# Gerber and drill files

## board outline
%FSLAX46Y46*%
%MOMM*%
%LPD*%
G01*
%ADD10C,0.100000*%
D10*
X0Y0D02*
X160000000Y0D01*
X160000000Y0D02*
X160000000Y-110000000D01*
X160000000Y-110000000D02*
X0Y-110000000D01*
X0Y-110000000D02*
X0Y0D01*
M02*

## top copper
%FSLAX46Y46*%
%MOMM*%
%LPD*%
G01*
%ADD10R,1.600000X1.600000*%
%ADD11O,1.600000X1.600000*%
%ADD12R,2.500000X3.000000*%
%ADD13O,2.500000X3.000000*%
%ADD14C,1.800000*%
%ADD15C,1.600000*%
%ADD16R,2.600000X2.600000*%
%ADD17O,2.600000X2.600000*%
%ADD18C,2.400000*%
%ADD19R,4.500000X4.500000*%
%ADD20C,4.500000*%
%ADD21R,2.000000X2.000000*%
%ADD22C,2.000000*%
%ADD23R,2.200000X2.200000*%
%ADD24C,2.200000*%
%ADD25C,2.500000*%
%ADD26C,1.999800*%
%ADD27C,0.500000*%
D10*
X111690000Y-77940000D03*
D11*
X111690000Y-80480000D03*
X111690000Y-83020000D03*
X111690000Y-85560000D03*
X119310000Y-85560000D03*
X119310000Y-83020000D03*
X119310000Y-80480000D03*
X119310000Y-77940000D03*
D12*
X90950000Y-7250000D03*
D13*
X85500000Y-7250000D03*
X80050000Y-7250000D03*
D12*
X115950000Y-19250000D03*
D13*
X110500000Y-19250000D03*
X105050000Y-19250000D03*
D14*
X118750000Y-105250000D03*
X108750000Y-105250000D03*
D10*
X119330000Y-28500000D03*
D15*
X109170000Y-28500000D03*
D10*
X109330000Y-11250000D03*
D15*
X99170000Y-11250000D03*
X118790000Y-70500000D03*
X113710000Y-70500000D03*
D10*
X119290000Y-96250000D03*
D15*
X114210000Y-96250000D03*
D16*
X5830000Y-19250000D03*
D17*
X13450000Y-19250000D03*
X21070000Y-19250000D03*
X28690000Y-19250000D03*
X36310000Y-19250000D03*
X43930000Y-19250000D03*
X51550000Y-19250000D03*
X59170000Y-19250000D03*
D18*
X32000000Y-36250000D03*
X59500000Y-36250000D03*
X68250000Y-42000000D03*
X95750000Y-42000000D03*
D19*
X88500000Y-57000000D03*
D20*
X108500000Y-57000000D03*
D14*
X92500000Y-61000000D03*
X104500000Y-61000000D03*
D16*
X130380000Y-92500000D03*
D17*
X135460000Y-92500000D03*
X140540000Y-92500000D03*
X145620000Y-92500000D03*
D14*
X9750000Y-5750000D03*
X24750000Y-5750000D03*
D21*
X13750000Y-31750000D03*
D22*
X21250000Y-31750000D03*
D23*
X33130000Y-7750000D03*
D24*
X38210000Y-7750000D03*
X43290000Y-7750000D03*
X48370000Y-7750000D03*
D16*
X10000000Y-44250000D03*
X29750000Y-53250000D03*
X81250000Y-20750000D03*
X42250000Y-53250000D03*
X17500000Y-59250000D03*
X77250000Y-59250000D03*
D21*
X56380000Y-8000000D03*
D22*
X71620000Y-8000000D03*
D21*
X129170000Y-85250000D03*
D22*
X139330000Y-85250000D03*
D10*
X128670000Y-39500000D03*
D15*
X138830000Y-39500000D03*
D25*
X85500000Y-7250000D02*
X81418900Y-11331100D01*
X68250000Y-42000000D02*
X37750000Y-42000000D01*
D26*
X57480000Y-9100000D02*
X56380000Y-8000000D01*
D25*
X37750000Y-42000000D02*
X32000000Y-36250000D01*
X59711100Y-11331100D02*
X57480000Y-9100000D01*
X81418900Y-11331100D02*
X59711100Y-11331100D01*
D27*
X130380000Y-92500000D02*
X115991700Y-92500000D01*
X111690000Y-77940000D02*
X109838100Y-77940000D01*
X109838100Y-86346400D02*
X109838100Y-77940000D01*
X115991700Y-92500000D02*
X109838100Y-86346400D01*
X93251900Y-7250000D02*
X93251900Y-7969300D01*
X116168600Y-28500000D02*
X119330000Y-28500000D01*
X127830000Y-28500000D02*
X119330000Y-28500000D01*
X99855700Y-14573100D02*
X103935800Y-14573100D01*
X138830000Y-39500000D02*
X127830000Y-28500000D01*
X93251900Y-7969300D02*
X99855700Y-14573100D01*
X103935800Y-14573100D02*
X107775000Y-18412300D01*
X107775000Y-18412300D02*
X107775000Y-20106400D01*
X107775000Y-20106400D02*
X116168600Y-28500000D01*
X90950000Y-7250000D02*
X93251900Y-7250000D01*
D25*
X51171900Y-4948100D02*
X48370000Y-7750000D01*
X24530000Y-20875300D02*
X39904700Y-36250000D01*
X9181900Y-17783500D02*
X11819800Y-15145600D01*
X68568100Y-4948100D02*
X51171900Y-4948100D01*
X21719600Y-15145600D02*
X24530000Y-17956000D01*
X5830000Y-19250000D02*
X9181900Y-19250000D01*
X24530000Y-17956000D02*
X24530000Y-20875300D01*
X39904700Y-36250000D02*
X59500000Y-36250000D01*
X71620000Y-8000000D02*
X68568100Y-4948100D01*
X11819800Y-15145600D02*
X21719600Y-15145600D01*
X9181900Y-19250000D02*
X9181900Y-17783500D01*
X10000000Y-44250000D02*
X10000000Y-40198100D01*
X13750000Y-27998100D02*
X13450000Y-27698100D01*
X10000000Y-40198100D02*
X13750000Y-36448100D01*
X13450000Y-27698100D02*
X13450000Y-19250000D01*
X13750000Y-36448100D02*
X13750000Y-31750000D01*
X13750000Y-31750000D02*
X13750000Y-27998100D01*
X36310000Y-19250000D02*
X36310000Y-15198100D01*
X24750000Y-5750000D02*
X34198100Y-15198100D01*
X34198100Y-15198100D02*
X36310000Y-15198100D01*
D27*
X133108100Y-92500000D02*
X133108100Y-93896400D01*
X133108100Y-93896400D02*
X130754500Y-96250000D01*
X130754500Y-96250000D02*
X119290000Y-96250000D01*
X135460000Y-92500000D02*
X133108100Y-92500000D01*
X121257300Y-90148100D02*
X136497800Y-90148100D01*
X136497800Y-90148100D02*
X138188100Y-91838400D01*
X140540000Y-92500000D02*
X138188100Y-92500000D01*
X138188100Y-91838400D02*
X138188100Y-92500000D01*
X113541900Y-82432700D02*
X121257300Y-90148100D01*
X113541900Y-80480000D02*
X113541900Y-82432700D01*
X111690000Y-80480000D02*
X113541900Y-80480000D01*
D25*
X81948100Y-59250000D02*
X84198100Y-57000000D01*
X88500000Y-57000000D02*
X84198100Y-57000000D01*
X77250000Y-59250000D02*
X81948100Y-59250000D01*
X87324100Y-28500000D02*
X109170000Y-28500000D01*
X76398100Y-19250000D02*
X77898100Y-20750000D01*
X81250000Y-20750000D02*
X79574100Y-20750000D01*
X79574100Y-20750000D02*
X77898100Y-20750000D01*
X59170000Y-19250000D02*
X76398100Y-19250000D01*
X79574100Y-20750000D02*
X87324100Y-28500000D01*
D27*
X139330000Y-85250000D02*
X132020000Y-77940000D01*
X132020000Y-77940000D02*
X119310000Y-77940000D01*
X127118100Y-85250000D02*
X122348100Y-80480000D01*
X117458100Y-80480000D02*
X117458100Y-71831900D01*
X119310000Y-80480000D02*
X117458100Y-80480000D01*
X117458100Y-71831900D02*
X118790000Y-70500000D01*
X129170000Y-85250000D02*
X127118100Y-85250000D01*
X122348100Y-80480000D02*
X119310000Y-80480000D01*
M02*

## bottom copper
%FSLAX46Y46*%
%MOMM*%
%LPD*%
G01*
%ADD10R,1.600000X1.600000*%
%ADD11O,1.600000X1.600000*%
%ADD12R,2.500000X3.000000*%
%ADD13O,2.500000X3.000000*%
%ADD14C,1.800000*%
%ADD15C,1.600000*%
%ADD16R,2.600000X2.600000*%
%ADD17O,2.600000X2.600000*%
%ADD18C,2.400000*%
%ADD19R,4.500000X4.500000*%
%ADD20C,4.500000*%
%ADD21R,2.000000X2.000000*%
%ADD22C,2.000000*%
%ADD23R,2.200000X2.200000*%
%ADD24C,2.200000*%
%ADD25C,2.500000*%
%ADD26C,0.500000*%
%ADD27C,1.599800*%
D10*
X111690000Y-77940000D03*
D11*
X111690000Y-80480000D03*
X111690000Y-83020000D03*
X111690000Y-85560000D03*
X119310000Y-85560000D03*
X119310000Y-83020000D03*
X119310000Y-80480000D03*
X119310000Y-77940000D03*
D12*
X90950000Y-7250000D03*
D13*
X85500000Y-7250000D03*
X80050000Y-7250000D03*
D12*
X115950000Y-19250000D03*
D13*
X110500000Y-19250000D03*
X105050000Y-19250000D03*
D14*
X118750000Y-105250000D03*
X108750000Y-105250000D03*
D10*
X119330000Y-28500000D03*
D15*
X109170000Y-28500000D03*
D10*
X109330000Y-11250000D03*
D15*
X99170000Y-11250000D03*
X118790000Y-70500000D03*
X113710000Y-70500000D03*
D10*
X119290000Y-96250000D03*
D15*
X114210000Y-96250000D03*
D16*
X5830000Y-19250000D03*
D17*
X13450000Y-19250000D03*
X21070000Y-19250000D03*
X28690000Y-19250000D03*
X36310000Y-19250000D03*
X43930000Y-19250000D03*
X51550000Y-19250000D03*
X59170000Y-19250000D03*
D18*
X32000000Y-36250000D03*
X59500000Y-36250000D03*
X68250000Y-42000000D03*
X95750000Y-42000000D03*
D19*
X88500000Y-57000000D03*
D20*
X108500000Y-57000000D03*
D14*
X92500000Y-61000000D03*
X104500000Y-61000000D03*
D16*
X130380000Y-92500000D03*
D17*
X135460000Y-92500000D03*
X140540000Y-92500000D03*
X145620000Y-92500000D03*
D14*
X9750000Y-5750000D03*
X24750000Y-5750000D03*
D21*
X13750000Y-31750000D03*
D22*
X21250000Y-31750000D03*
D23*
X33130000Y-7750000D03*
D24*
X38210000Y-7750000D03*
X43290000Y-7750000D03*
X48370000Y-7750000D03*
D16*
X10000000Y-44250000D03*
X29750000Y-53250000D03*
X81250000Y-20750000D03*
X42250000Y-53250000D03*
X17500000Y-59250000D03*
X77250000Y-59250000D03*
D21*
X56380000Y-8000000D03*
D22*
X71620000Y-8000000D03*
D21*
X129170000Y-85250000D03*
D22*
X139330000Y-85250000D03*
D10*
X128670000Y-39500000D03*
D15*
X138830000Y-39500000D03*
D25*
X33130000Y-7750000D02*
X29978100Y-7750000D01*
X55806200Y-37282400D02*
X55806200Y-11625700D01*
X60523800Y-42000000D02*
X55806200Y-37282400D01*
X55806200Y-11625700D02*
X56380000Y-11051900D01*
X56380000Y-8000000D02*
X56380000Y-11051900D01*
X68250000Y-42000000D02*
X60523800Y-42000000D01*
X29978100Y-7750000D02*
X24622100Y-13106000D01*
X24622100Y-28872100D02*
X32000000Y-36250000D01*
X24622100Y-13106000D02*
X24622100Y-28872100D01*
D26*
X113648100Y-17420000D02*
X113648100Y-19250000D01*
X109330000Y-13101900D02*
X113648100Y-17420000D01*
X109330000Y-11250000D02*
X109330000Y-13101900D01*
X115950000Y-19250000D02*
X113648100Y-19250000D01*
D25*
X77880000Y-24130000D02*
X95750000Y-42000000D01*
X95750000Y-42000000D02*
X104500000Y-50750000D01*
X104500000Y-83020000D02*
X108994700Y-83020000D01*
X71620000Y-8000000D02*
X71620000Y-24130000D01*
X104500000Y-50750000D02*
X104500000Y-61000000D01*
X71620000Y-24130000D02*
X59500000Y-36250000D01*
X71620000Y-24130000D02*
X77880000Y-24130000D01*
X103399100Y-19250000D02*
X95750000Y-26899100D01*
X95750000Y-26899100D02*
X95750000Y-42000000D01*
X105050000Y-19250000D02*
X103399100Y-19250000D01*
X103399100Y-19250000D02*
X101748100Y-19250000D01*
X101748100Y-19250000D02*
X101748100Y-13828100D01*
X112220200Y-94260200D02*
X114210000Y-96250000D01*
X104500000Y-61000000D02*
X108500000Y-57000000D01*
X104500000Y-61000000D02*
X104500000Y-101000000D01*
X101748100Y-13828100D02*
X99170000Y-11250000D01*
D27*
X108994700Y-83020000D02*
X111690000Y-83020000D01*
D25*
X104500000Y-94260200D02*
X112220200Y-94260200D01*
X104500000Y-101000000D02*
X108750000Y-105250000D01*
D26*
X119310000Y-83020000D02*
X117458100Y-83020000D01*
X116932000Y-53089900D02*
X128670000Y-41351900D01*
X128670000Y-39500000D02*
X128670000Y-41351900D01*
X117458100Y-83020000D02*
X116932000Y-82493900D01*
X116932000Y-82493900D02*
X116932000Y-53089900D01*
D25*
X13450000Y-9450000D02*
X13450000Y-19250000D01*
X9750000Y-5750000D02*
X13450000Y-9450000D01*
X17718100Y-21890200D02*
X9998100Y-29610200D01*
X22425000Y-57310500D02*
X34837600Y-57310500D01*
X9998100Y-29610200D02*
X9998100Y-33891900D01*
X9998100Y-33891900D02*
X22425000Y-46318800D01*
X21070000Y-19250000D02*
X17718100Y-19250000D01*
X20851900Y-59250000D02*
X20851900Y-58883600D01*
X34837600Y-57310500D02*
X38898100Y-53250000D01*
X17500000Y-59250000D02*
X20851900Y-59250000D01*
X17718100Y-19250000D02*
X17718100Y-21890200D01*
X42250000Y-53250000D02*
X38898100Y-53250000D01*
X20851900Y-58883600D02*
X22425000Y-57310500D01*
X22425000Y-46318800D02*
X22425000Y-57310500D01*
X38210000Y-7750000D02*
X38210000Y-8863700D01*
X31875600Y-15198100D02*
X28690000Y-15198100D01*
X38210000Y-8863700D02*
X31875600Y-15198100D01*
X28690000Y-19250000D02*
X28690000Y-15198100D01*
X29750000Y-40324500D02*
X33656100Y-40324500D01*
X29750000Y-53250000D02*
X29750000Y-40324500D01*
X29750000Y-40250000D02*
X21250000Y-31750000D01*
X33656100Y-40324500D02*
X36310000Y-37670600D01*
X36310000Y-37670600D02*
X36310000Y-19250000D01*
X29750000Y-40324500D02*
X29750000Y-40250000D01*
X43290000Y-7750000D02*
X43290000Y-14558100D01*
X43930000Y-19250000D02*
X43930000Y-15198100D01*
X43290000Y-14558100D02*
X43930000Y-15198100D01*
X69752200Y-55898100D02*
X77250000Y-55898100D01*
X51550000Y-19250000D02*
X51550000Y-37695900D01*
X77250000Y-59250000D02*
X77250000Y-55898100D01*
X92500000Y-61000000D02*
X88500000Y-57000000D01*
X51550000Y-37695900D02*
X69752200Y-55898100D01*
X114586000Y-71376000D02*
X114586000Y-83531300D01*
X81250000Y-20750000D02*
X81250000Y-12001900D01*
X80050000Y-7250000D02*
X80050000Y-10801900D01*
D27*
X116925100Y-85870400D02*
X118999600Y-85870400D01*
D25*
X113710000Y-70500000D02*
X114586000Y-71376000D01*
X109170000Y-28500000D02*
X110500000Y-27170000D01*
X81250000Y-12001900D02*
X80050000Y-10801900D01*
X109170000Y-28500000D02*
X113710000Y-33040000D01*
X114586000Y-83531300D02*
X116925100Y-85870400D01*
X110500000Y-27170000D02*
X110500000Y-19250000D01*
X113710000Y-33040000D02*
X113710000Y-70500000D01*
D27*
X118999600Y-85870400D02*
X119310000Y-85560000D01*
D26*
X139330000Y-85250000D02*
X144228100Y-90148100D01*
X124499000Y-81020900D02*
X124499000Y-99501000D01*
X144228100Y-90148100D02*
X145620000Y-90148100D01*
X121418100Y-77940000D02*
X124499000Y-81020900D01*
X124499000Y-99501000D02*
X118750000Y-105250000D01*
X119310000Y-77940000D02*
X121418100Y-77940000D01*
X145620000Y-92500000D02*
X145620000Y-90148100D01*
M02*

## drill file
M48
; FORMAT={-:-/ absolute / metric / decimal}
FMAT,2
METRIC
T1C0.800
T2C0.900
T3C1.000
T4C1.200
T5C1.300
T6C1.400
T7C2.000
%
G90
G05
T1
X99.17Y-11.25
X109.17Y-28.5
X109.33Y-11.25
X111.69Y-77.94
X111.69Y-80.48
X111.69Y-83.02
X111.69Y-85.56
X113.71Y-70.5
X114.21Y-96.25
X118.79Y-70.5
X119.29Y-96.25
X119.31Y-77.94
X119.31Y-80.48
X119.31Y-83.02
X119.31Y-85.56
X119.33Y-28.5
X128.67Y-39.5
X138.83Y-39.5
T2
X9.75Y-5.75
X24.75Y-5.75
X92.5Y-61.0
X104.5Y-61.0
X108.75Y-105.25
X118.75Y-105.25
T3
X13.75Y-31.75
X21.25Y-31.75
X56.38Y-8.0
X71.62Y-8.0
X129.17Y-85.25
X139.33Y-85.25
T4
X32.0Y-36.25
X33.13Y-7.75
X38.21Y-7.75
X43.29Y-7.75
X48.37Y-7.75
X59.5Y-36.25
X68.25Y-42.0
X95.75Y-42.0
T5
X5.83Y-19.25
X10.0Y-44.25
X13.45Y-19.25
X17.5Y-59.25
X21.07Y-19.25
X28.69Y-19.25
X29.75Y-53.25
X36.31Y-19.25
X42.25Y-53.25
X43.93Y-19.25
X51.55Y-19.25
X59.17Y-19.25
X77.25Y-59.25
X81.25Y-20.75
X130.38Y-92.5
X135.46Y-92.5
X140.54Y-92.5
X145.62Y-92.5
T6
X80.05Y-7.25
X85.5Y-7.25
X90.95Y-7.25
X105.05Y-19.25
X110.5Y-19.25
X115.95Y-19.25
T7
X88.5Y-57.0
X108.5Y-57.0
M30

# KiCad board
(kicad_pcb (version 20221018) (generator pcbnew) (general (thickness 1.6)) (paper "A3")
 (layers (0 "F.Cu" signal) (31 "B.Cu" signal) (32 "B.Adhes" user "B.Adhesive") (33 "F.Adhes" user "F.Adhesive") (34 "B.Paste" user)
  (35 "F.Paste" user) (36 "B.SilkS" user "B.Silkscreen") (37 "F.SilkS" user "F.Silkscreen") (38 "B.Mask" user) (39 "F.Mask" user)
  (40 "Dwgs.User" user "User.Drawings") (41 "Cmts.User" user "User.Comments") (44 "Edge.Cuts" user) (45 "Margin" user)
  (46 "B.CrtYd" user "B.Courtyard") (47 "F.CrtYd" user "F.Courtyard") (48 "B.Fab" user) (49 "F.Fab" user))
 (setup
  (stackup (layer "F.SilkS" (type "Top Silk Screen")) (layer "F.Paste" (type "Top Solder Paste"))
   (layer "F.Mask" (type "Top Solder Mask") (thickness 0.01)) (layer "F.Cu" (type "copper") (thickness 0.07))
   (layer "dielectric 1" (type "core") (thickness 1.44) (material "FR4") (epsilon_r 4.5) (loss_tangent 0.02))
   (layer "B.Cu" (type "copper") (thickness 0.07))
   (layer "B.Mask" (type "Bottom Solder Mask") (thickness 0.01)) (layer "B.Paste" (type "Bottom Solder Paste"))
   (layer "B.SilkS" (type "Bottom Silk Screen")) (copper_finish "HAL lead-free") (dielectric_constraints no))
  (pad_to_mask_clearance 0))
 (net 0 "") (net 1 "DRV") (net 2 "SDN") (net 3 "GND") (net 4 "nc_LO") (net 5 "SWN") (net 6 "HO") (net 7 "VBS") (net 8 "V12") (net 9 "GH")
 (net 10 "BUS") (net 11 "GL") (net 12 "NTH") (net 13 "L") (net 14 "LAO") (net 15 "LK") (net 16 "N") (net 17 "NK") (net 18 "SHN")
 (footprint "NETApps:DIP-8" (layer "F.Cu") (at 115.5 81.75)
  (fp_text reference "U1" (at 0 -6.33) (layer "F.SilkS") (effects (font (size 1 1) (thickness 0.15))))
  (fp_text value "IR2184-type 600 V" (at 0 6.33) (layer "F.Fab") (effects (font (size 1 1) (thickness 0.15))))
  (pad "1" thru_hole rect (at -3.81 -3.81) (size 1.6 1.6) (drill 0.8) (layers "*.Cu" "*.Mask") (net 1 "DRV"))
  (pad "2" thru_hole oval (at -3.81 -1.27) (size 1.6 1.6) (drill 0.8) (layers "*.Cu" "*.Mask") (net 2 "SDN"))
  (pad "3" thru_hole oval (at -3.81 1.27) (size 1.6 1.6) (drill 0.8) (layers "*.Cu" "*.Mask") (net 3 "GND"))
  (pad "4" thru_hole oval (at -3.81 3.81) (size 1.6 1.6) (drill 0.8) (layers "*.Cu" "*.Mask") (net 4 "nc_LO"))
  (pad "5" thru_hole oval (at 3.81 3.81) (size 1.6 1.6) (drill 0.8) (layers "*.Cu" "*.Mask") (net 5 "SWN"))
  (pad "6" thru_hole oval (at 3.81 1.27) (size 1.6 1.6) (drill 0.8) (layers "*.Cu" "*.Mask") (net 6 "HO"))
  (pad "7" thru_hole oval (at 3.81 -1.27) (size 1.6 1.6) (drill 0.8) (layers "*.Cu" "*.Mask") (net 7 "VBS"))
  (pad "8" thru_hole oval (at 3.81 -3.81) (size 1.6 1.6) (drill 0.8) (layers "*.Cu" "*.Mask") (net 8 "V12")))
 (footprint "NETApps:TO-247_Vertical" (layer "F.Cu") (at 85.5 7.25 180)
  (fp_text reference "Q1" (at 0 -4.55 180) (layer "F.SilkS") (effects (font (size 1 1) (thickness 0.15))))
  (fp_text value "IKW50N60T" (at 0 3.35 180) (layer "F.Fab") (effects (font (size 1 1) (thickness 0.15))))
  (pad "1" thru_hole rect (at -5.45 0) (size 2.5 3) (drill 1.4) (layers "*.Cu" "*.Mask") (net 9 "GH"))
  (pad "2" thru_hole oval (at 0 0) (size 2.5 3) (drill 1.4) (layers "*.Cu" "*.Mask") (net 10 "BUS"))
  (pad "3" thru_hole oval (at 5.45 0) (size 2.5 3) (drill 1.4) (layers "*.Cu" "*.Mask") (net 5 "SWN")))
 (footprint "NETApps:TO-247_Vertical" (layer "F.Cu") (at 110.5 19.25 180)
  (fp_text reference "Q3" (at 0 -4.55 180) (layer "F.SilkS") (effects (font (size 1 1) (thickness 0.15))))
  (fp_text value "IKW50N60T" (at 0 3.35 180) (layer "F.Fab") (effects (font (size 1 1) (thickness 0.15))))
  (pad "1" thru_hole rect (at -5.45 0) (size 2.5 3) (drill 1.4) (layers "*.Cu" "*.Mask") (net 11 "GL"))
  (pad "2" thru_hole oval (at 0 0) (size 2.5 3) (drill 1.4) (layers "*.Cu" "*.Mask") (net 5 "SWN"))
  (pad "3" thru_hole oval (at 5.45 0) (size 2.5 3) (drill 1.4) (layers "*.Cu" "*.Mask") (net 3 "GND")))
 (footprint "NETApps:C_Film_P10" (layer "F.Cu") (at 113.75 105.25 180)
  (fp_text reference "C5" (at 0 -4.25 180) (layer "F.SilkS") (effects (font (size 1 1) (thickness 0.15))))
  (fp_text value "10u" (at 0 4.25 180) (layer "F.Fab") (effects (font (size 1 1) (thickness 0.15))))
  (pad "1" thru_hole circle (at -5 0) (size 1.8 1.8) (drill 0.9) (layers "*.Cu" "*.Mask") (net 8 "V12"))
  (pad "2" thru_hole circle (at 5 0) (size 1.8 1.8) (drill 0.9) (layers "*.Cu" "*.Mask") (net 3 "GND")))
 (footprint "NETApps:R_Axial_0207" (layer "F.Cu") (at 114.25 28.5 180)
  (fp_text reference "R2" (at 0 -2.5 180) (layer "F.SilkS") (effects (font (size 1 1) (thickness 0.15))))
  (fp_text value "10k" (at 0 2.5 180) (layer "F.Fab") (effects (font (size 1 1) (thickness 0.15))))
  (pad "1" thru_hole rect (at -5.08 0) (size 1.6 1.6) (drill 0.8) (layers "*.Cu" "*.Mask") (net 9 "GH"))
  (pad "2" thru_hole circle (at 5.08 0) (size 1.6 1.6) (drill 0.8) (layers "*.Cu" "*.Mask") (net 5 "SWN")))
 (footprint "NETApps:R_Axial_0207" (layer "F.Cu") (at 104.25 11.25 180)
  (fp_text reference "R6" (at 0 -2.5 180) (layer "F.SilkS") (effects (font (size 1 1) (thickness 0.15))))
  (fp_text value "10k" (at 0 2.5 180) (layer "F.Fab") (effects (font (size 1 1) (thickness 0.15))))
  (pad "1" thru_hole rect (at -5.08 0) (size 1.6 1.6) (drill 0.8) (layers "*.Cu" "*.Mask") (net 11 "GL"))
  (pad "2" thru_hole circle (at 5.08 0) (size 1.6 1.6) (drill 0.8) (layers "*.Cu" "*.Mask") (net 3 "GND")))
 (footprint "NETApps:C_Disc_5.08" (layer "F.Cu") (at 116.25 70.5 180)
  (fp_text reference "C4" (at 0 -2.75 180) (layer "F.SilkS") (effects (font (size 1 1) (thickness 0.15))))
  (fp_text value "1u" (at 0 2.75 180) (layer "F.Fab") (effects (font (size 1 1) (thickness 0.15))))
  (pad "1" thru_hole circle (at -2.54 0) (size 1.6 1.6) (drill 0.8) (layers "*.Cu" "*.Mask") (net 7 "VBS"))
  (pad "2" thru_hole circle (at 2.54 0) (size 1.6 1.6) (drill 0.8) (layers "*.Cu" "*.Mask") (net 5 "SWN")))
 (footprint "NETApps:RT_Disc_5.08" (layer "F.Cu") (at 116.75 96.25 180)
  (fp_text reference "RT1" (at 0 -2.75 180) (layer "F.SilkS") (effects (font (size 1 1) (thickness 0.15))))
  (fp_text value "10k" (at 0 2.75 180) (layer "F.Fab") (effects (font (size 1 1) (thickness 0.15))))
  (pad "1" thru_hole rect (at -2.54 0) (size 1.6 1.6) (drill 0.8) (layers "*.Cu" "*.Mask") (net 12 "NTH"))
  (pad "2" thru_hole circle (at 2.54 0) (size 1.6 1.6) (drill 0.8) (layers "*.Cu" "*.Mask") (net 3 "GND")))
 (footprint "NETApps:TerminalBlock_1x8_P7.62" (layer "F.Cu") (at 32.5 19.25)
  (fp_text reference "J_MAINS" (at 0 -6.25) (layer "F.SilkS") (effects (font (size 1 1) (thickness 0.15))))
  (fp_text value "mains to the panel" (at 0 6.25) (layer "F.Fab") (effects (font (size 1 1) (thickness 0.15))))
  (pad "1" thru_hole rect (at -26.67 0) (size 2.6 2.6) (drill 1.3) (layers "*.Cu" "*.Mask") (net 3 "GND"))
  (pad "2" thru_hole oval (at -19.05 0) (size 2.6 2.6) (drill 1.3) (layers "*.Cu" "*.Mask") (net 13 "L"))
  (pad "3" thru_hole oval (at -11.43 0) (size 2.6 2.6) (drill 1.3) (layers "*.Cu" "*.Mask") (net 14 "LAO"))
  (pad "4" thru_hole oval (at -3.81 0) (size 2.6 2.6) (drill 1.3) (layers "*.Cu" "*.Mask") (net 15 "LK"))
  (pad "5" thru_hole oval (at 3.81 0) (size 2.6 2.6) (drill 1.3) (layers "*.Cu" "*.Mask") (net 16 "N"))
  (pad "6" thru_hole oval (at 11.43 0) (size 2.6 2.6) (drill 1.3) (layers "*.Cu" "*.Mask") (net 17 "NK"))
  (pad "7" thru_hole oval (at 19.05 0) (size 2.6 2.6) (drill 1.3) (layers "*.Cu" "*.Mask") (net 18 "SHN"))
  (pad "8" thru_hole oval (at 26.67 0) (size 2.6 2.6) (drill 1.3) (layers "*.Cu" "*.Mask") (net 5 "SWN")))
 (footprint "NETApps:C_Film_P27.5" (layer "F.Cu") (at 45.75 36.25)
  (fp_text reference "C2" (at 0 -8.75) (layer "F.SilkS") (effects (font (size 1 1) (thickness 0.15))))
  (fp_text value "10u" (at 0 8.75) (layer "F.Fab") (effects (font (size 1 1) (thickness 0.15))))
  (pad "1" thru_hole circle (at -13.75 0) (size 2.4 2.4) (drill 1.2) (layers "*.Cu" "*.Mask") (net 10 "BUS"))
  (pad "2" thru_hole circle (at 13.75 0) (size 2.4 2.4) (drill 1.2) (layers "*.Cu" "*.Mask") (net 3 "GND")))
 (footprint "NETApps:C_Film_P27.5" (layer "F.Cu") (at 82 42)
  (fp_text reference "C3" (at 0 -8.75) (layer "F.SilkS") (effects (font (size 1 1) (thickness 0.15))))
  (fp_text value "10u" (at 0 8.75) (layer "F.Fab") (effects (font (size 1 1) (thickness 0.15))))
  (pad "1" thru_hole circle (at -13.75 0) (size 2.4 2.4) (drill 1.2) (layers "*.Cu" "*.Mask") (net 10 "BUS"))
  (pad "2" thru_hole circle (at 13.75 0) (size 2.4 2.4) (drill 1.2) (layers "*.Cu" "*.Mask") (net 3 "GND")))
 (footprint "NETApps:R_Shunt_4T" (layer "F.Cu") (at 98.5 57)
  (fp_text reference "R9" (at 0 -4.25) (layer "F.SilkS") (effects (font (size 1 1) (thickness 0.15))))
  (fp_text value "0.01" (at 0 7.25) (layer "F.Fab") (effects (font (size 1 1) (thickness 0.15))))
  (pad "1" thru_hole rect (at -10 0) (size 4.5 4.5) (drill 2) (layers "*.Cu" "*.Mask") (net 18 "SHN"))
  (pad "2" thru_hole circle (at 10 0) (size 4.5 4.5) (drill 2) (layers "*.Cu" "*.Mask") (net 3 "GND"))
  (pad "3" thru_hole circle (at -6 4) (size 1.8 1.8) (drill 0.9) (layers "*.Cu" "*.Mask") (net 18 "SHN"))
  (pad "4" thru_hole circle (at 6 4) (size 1.8 1.8) (drill 0.9) (layers "*.Cu" "*.Mask") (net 3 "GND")))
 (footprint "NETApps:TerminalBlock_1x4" (layer "F.Cu") (at 138 92.5)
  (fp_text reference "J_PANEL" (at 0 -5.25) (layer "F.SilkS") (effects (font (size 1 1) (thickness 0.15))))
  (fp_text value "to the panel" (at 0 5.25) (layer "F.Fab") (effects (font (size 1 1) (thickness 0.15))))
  (pad "1" thru_hole rect (at -7.62 0) (size 2.6 2.6) (drill 1.3) (layers "*.Cu" "*.Mask") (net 1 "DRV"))
  (pad "2" thru_hole oval (at -2.54 0) (size 2.6 2.6) (drill 1.3) (layers "*.Cu" "*.Mask") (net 12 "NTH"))
  (pad "3" thru_hole oval (at 2.54 0) (size 2.6 2.6) (drill 1.3) (layers "*.Cu" "*.Mask") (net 2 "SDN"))
  (pad "4" thru_hole oval (at 7.62 0) (size 2.6 2.6) (drill 1.3) (layers "*.Cu" "*.Mask") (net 8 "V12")))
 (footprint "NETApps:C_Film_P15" (layer "F.Cu") (at 17.25 5.75)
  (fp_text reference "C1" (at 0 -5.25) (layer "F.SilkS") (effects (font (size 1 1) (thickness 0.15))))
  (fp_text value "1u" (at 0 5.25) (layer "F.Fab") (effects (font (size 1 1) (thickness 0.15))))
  (pad "1" thru_hole circle (at -7.5 0) (size 1.8 1.8) (drill 0.9) (layers "*.Cu" "*.Mask") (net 13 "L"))
  (pad "2" thru_hole circle (at 7.5 0) (size 1.8 1.8) (drill 0.9) (layers "*.Cu" "*.Mask") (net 16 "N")))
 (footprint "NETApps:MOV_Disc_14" (layer "F.Cu") (at 17.5 31.75)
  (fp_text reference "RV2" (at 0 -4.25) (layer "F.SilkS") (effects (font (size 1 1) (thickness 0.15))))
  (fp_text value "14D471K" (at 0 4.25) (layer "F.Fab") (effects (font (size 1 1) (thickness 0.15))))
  (pad "1" thru_hole rect (at -3.75 0) (size 2 2) (drill 1) (layers "*.Cu" "*.Mask") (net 13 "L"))
  (pad "2" thru_hole circle (at 3.75 0) (size 2 2) (drill 1) (layers "*.Cu" "*.Mask") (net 16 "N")))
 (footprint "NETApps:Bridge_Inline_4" (layer "F.Cu") (at 40.75 7.75)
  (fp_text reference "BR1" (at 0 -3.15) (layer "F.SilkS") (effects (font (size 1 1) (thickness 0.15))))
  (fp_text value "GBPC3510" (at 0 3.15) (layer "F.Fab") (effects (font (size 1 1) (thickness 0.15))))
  (pad "1" thru_hole rect (at -7.62 0) (size 2.2 2.2) (drill 1.2) (layers "*.Cu" "*.Mask") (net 10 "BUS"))
  (pad "2" thru_hole circle (at -2.54 0) (size 2.2 2.2) (drill 1.2) (layers "*.Cu" "*.Mask") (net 15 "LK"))
  (pad "3" thru_hole circle (at 2.54 0) (size 2.2 2.2) (drill 1.2) (layers "*.Cu" "*.Mask") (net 17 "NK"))
  (pad "4" thru_hole circle (at 7.62 0) (size 2.2 2.2) (drill 1.2) (layers "*.Cu" "*.Mask") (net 3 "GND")))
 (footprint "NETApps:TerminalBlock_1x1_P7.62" (layer "F.Cu") (at 10 44.25)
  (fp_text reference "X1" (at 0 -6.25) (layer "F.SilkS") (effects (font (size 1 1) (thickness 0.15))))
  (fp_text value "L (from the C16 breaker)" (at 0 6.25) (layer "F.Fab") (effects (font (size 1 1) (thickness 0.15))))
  (pad "1" thru_hole rect (at 0 0) (size 2.6 2.6) (drill 1.3) (layers "*.Cu" "*.Mask") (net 13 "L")))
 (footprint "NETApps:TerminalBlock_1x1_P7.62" (layer "F.Cu") (at 29.75 53.25)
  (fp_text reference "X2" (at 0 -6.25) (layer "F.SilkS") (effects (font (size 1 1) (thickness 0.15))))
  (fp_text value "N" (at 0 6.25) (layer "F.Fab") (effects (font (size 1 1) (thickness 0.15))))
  (pad "1" thru_hole rect (at 0 0) (size 2.6 2.6) (drill 1.3) (layers "*.Cu" "*.Mask") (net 16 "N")))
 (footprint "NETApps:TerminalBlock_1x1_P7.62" (layer "F.Cu") (at 81.25 20.75)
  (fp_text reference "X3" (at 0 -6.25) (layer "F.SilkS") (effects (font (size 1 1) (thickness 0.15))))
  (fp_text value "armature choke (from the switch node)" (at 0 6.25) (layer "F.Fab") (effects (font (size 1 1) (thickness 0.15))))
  (pad "1" thru_hole rect (at 0 0) (size 2.6 2.6) (drill 1.3) (layers "*.Cu" "*.Mask") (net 5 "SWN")))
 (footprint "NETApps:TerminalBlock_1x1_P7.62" (layer "F.Cu") (at 42.25 53.25)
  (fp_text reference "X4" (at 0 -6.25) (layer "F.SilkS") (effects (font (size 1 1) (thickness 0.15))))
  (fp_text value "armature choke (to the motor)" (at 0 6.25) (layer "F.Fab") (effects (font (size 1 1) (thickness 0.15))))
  (pad "1" thru_hole rect (at 0 0) (size 2.6 2.6) (drill 1.3) (layers "*.Cu" "*.Mask") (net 14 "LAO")))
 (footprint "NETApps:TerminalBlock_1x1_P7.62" (layer "F.Cu") (at 17.5 59.25)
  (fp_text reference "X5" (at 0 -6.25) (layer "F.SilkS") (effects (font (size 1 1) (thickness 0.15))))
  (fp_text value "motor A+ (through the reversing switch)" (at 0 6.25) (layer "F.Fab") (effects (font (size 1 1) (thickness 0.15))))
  (pad "1" thru_hole rect (at 0 0) (size 2.6 2.6) (drill 1.3) (layers "*.Cu" "*.Mask") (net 14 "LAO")))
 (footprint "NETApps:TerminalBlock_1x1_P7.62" (layer "F.Cu") (at 77.25 59.25)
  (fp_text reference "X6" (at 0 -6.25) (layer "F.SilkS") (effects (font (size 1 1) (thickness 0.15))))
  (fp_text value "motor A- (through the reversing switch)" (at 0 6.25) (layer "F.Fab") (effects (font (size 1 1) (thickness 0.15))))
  (pad "1" thru_hole rect (at 0 0) (size 2.6 2.6) (drill 1.3) (layers "*.Cu" "*.Mask") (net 18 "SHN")))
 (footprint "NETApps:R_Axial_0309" (layer "F.Cu") (at 64 8)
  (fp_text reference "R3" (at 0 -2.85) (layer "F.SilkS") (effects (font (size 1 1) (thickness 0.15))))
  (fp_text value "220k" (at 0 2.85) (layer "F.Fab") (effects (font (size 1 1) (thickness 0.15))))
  (pad "1" thru_hole rect (at -7.62 0) (size 2 2) (drill 1) (layers "*.Cu" "*.Mask") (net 10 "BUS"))
  (pad "2" thru_hole circle (at 7.62 0) (size 2 2) (drill 1) (layers "*.Cu" "*.Mask") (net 3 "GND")))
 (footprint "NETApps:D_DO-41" (layer "F.Cu") (at 134.25 85.25)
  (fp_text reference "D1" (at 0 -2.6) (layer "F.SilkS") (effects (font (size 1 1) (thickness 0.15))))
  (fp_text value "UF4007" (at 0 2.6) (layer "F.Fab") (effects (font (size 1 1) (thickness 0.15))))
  (pad "1" thru_hole rect (at -5.08 0) (size 2 2) (drill 1) (layers "*.Cu" "*.Mask") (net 7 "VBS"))
  (pad "2" thru_hole circle (at 5.08 0) (size 2 2) (drill 1) (layers "*.Cu" "*.Mask") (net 8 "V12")))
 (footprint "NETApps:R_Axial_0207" (layer "F.Cu") (at 133.75 39.5)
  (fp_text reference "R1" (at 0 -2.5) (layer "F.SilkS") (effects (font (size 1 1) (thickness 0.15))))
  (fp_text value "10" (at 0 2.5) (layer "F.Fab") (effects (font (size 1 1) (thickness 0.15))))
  (pad "1" thru_hole rect (at -5.08 0) (size 1.6 1.6) (drill 0.8) (layers "*.Cu" "*.Mask") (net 6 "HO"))
  (pad "2" thru_hole circle (at 5.08 0) (size 1.6 1.6) (drill 0.8) (layers "*.Cu" "*.Mask") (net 9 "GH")))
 (gr_line (start 0 0) (end 160 0) (stroke (width 0.1) (type solid)) (layer "Edge.Cuts"))
 (gr_line (start 160 0) (end 160 110) (stroke (width 0.1) (type solid)) (layer "Edge.Cuts"))
 (gr_line (start 160 110) (end 0 110) (stroke (width 0.1) (type solid)) (layer "Edge.Cuts"))
 (gr_line (start 0 110) (end 0 0) (stroke (width 0.1) (type solid)) (layer "Edge.Cuts"))
 (segment (start 85.5 7.25) (end 81.4189 11.3311) (width 2.5) (layer "F.Cu") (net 10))
 (segment locked (start 68.25 42) (end 37.75 42) (width 2.5) (layer "F.Cu") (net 10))
 (segment (start 57.48 9.1) (end 56.38 8) (width 1.9998) (layer "F.Cu") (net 10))
 (segment locked (start 37.75 42) (end 32 36.25) (width 2.5) (layer "F.Cu") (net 10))
 (segment (start 59.7111 11.3311) (end 57.48 9.1) (width 2.5) (layer "F.Cu") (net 10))
 (segment (start 81.4189 11.3311) (end 59.7111 11.3311) (width 2.5) (layer "F.Cu") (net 10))
 (segment locked (start 33.13 7.75) (end 29.9781 7.75) (width 2.5) (layer "B.Cu") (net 10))
 (segment locked (start 55.8062 37.2824) (end 55.8062 11.6257) (width 2.5) (layer "B.Cu") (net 10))
 (segment locked (start 60.5238 42) (end 55.8062 37.2824) (width 2.5) (layer "B.Cu") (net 10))
 (segment locked (start 55.8062 11.6257) (end 56.38 11.0519) (width 2.5) (layer "B.Cu") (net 10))
 (segment locked (start 56.38 8) (end 56.38 11.0519) (width 2.5) (layer "B.Cu") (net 10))
 (segment locked (start 68.25 42) (end 60.5238 42) (width 2.5) (layer "B.Cu") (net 10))
 (segment locked (start 29.9781 7.75) (end 24.6221 13.106) (width 2.5) (layer "B.Cu") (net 10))
 (segment locked (start 24.6221 28.8721) (end 32 36.25) (width 2.5) (layer "B.Cu") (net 10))
 (segment locked (start 24.6221 13.106) (end 24.6221 28.8721) (width 2.5) (layer "B.Cu") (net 10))
 (segment (start 130.38 92.5) (end 115.9917 92.5) (width 0.5) (layer "F.Cu") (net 1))
 (segment (start 111.69 77.94) (end 109.8381 77.94) (width 0.5) (layer "F.Cu") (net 1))
 (segment (start 109.8381 86.3464) (end 109.8381 77.94) (width 0.5) (layer "F.Cu") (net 1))
 (segment (start 115.9917 92.5) (end 109.8381 86.3464) (width 0.5) (layer "F.Cu") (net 1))
 (segment (start 93.2519 7.25) (end 93.2519 7.9693) (width 0.5) (layer "F.Cu") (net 9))
 (segment (start 116.1686 28.5) (end 119.33 28.5) (width 0.5) (layer "F.Cu") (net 9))
 (segment (start 127.83 28.5) (end 119.33 28.5) (width 0.5) (layer "F.Cu") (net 9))
 (segment (start 99.8557 14.5731) (end 103.9358 14.5731) (width 0.5) (layer "F.Cu") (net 9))
 (segment (start 138.83 39.5) (end 127.83 28.5) (width 0.5) (layer "F.Cu") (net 9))
 (segment (start 93.2519 7.9693) (end 99.8557 14.5731) (width 0.5) (layer "F.Cu") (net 9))
 (segment (start 103.9358 14.5731) (end 107.775 18.4123) (width 0.5) (layer "F.Cu") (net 9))
 (segment (start 107.775 18.4123) (end 107.775 20.1064) (width 0.5) (layer "F.Cu") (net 9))
 (segment (start 107.775 20.1064) (end 116.1686 28.5) (width 0.5) (layer "F.Cu") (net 9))
 (segment (start 90.95 7.25) (end 93.2519 7.25) (width 0.5) (layer "F.Cu") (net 9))
 (segment (start 113.6481 17.42) (end 113.6481 19.25) (width 0.5) (layer "B.Cu") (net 11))
 (segment (start 109.33 13.1019) (end 113.6481 17.42) (width 0.5) (layer "B.Cu") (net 11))
 (segment (start 109.33 11.25) (end 109.33 13.1019) (width 0.5) (layer "B.Cu") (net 11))
 (segment (start 115.95 19.25) (end 113.6481 19.25) (width 0.5) (layer "B.Cu") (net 11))
 (segment locked (start 51.1719 4.9481) (end 48.37 7.75) (width 2.5) (layer "F.Cu") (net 3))
 (segment locked (start 24.53 20.8753) (end 39.9047 36.25) (width 2.5) (layer "F.Cu") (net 3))
 (segment locked (start 9.1819 17.7835) (end 11.8198 15.1456) (width 2.5) (layer "F.Cu") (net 3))
 (segment locked (start 68.5681 4.9481) (end 51.1719 4.9481) (width 2.5) (layer "F.Cu") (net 3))
 (segment locked (start 21.7196 15.1456) (end 24.53 17.956) (width 2.5) (layer "F.Cu") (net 3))
 (segment locked (start 5.83 19.25) (end 9.1819 19.25) (width 2.5) (layer "F.Cu") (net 3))
 (segment locked (start 24.53 17.956) (end 24.53 20.8753) (width 2.5) (layer "F.Cu") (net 3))
 (segment locked (start 39.9047 36.25) (end 59.5 36.25) (width 2.5) (layer "F.Cu") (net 3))
 (segment locked (start 71.62 8) (end 68.5681 4.9481) (width 2.5) (layer "F.Cu") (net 3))
 (segment locked (start 11.8198 15.1456) (end 21.7196 15.1456) (width 2.5) (layer "F.Cu") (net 3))
 (segment locked (start 9.1819 19.25) (end 9.1819 17.7835) (width 2.5) (layer "F.Cu") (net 3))
 (segment locked (start 77.88 24.13) (end 95.75 42) (width 2.5) (layer "B.Cu") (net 3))
 (segment locked (start 95.75 42) (end 104.5 50.75) (width 2.5) (layer "B.Cu") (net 3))
 (segment (start 104.5 83.02) (end 108.9947 83.02) (width 2.5) (layer "B.Cu") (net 3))
 (segment locked (start 71.62 8) (end 71.62 24.13) (width 2.5) (layer "B.Cu") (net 3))
 (segment locked (start 104.5 50.75) (end 104.5 61) (width 2.5) (layer "B.Cu") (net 3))
 (segment locked (start 71.62 24.13) (end 59.5 36.25) (width 2.5) (layer "B.Cu") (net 3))
 (segment locked (start 71.62 24.13) (end 77.88 24.13) (width 2.5) (layer "B.Cu") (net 3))
 (segment locked (start 103.3991 19.25) (end 95.75 26.8991) (width 2.5) (layer "B.Cu") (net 3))
 (segment locked (start 95.75 26.8991) (end 95.75 42) (width 2.5) (layer "B.Cu") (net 3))
 (segment locked (start 105.05 19.25) (end 103.3991 19.25) (width 2.5) (layer "B.Cu") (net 3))
 (segment locked (start 103.3991 19.25) (end 101.7481 19.25) (width 2.5) (layer "B.Cu") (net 3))
 (segment locked (start 101.7481 19.25) (end 101.7481 13.8281) (width 2.5) (layer "B.Cu") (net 3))
 (segment (start 112.2202 94.2602) (end 114.21 96.25) (width 2.5) (layer "B.Cu") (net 3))
 (segment locked (start 104.5 61) (end 108.5 57) (width 2.5) (layer "B.Cu") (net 3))
 (segment locked (start 104.5 61) (end 104.5 101) (width 2.5) (layer "B.Cu") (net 3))
 (segment locked (start 101.7481 13.8281) (end 99.17 11.25) (width 2.5) (layer "B.Cu") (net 3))
 (segment (start 108.9947 83.02) (end 111.69 83.02) (width 1.5998) (layer "B.Cu") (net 3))
 (segment (start 104.5 94.2602) (end 112.2202 94.2602) (width 2.5) (layer "B.Cu") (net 3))
 (segment locked (start 104.5 101) (end 108.75 105.25) (width 2.5) (layer "B.Cu") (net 3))
 (segment (start 119.31 83.02) (end 117.4581 83.02) (width 0.5) (layer "B.Cu") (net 6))
 (segment (start 116.932 53.0899) (end 128.67 41.3519) (width 0.5) (layer "B.Cu") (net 6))
 (segment (start 128.67 39.5) (end 128.67 41.3519) (width 0.5) (layer "B.Cu") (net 6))
 (segment (start 117.4581 83.02) (end 116.932 82.4939) (width 0.5) (layer "B.Cu") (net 6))
 (segment (start 116.932 82.4939) (end 116.932 53.0899) (width 0.5) (layer "B.Cu") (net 6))
 (segment locked (start 10 44.25) (end 10 40.1981) (width 2.5) (layer "F.Cu") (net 13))
 (segment locked (start 13.75 27.9981) (end 13.45 27.6981) (width 2.5) (layer "F.Cu") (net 13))
 (segment locked (start 10 40.1981) (end 13.75 36.4481) (width 2.5) (layer "F.Cu") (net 13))
 (segment locked (start 13.45 27.6981) (end 13.45 19.25) (width 2.5) (layer "F.Cu") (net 13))
 (segment locked (start 13.75 36.4481) (end 13.75 31.75) (width 2.5) (layer "F.Cu") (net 13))
 (segment locked (start 13.75 31.75) (end 13.75 27.9981) (width 2.5) (layer "F.Cu") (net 13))
 (segment locked (start 13.45 9.45) (end 13.45 19.25) (width 2.5) (layer "B.Cu") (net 13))
 (segment locked (start 9.75 5.75) (end 13.45 9.45) (width 2.5) (layer "B.Cu") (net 13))
 (segment locked (start 17.7181 21.8902) (end 9.9981 29.6102) (width 2.5) (layer "B.Cu") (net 14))
 (segment locked (start 22.425 57.3105) (end 34.8376 57.3105) (width 2.5) (layer "B.Cu") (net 14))
 (segment locked (start 9.9981 29.6102) (end 9.9981 33.8919) (width 2.5) (layer "B.Cu") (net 14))
 (segment locked (start 9.9981 33.8919) (end 22.425 46.3188) (width 2.5) (layer "B.Cu") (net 14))
 (segment locked (start 21.07 19.25) (end 17.7181 19.25) (width 2.5) (layer "B.Cu") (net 14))
 (segment locked (start 20.8519 59.25) (end 20.8519 58.8836) (width 2.5) (layer "B.Cu") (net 14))
 (segment locked (start 34.8376 57.3105) (end 38.8981 53.25) (width 2.5) (layer "B.Cu") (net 14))
 (segment locked (start 17.5 59.25) (end 20.8519 59.25) (width 2.5) (layer "B.Cu") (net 14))
 (segment locked (start 17.7181 19.25) (end 17.7181 21.8902) (width 2.5) (layer "B.Cu") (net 14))
 (segment locked (start 42.25 53.25) (end 38.8981 53.25) (width 2.5) (layer "B.Cu") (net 14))
 (segment locked (start 20.8519 58.8836) (end 22.425 57.3105) (width 2.5) (layer "B.Cu") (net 14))
 (segment locked (start 22.425 46.3188) (end 22.425 57.3105) (width 2.5) (layer "B.Cu") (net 14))
 (segment locked (start 38.21 7.75) (end 38.21 8.8637) (width 2.5) (layer "B.Cu") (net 15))
 (segment locked (start 31.8756 15.1981) (end 28.69 15.1981) (width 2.5) (layer "B.Cu") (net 15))
 (segment locked (start 38.21 8.8637) (end 31.8756 15.1981) (width 2.5) (layer "B.Cu") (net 15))
 (segment locked (start 28.69 19.25) (end 28.69 15.1981) (width 2.5) (layer "B.Cu") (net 15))
 (segment locked (start 36.31 19.25) (end 36.31 15.1981) (width 2.5) (layer "F.Cu") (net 16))
 (segment locked (start 24.75 5.75) (end 34.1981 15.1981) (width 2.5) (layer "F.Cu") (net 16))
 (segment locked (start 34.1981 15.1981) (end 36.31 15.1981) (width 2.5) (layer "F.Cu") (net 16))
 (segment locked (start 29.75 40.3245) (end 33.6561 40.3245) (width 2.5) (layer "B.Cu") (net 16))
 (segment locked (start 29.75 53.25) (end 29.75 40.3245) (width 2.5) (layer "B.Cu") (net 16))
 (segment locked (start 29.75 40.25) (end 21.25 31.75) (width 2.5) (layer "B.Cu") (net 16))
 (segment locked (start 33.6561 40.3245) (end 36.31 37.6706) (width 2.5) (layer "B.Cu") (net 16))
 (segment locked (start 36.31 37.6706) (end 36.31 19.25) (width 2.5) (layer "B.Cu") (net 16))
 (segment locked (start 29.75 40.3245) (end 29.75 40.25) (width 2.5) (layer "B.Cu") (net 16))
 (segment locked (start 43.29 7.75) (end 43.29 14.5581) (width 2.5) (layer "B.Cu") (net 17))
 (segment locked (start 43.93 19.25) (end 43.93 15.1981) (width 2.5) (layer "B.Cu") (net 17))
 (segment locked (start 43.29 14.5581) (end 43.93 15.1981) (width 2.5) (layer "B.Cu") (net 17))
 (segment (start 133.1081 92.5) (end 133.1081 93.8964) (width 0.5) (layer "F.Cu") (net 12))
 (segment (start 133.1081 93.8964) (end 130.7545 96.25) (width 0.5) (layer "F.Cu") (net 12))
 (segment (start 130.7545 96.25) (end 119.29 96.25) (width 0.5) (layer "F.Cu") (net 12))
 (segment (start 135.46 92.5) (end 133.1081 92.5) (width 0.5) (layer "F.Cu") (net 12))
 (segment (start 121.2573 90.1481) (end 136.4978 90.1481) (width 0.5) (layer "F.Cu") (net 2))
 (segment (start 136.4978 90.1481) (end 138.1881 91.8384) (width 0.5) (layer "F.Cu") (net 2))
 (segment (start 140.54 92.5) (end 138.1881 92.5) (width 0.5) (layer "F.Cu") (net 2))
 (segment (start 138.1881 91.8384) (end 138.1881 92.5) (width 0.5) (layer "F.Cu") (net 2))
 (segment (start 113.5419 82.4327) (end 121.2573 90.1481) (width 0.5) (layer "F.Cu") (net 2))
 (segment (start 113.5419 80.48) (end 113.5419 82.4327) (width 0.5) (layer "F.Cu") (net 2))
 (segment (start 111.69 80.48) (end 113.5419 80.48) (width 0.5) (layer "F.Cu") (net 2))
 (segment locked (start 81.9481 59.25) (end 84.1981 57) (width 2.5) (layer "F.Cu") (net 18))
 (segment locked (start 88.5 57) (end 84.1981 57) (width 2.5) (layer "F.Cu") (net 18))
 (segment locked (start 77.25 59.25) (end 81.9481 59.25) (width 2.5) (layer "F.Cu") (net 18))
 (segment locked (start 69.7522 55.8981) (end 77.25 55.8981) (width 2.5) (layer "B.Cu") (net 18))
 (segment locked (start 51.55 19.25) (end 51.55 37.6959) (width 2.5) (layer "B.Cu") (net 18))
 (segment locked (start 77.25 59.25) (end 77.25 55.8981) (width 2.5) (layer "B.Cu") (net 18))
 (segment locked (start 92.5 61) (end 88.5 57) (width 2.5) (layer "B.Cu") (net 18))
 (segment locked (start 51.55 37.6959) (end 69.7522 55.8981) (width 2.5) (layer "B.Cu") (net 18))
 (segment locked (start 87.3241 28.5) (end 109.17 28.5) (width 2.5) (layer "F.Cu") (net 5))
 (segment locked (start 76.3981 19.25) (end 77.8981 20.75) (width 2.5) (layer "F.Cu") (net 5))
 (segment locked (start 81.25 20.75) (end 79.5741 20.75) (width 2.5) (layer "F.Cu") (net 5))
 (segment locked (start 79.5741 20.75) (end 77.8981 20.75) (width 2.5) (layer "F.Cu") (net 5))
 (segment locked (start 59.17 19.25) (end 76.3981 19.25) (width 2.5) (layer "F.Cu") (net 5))
 (segment locked (start 79.5741 20.75) (end 87.3241 28.5) (width 2.5) (layer "F.Cu") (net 5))
 (segment (start 114.586 71.376) (end 114.586 83.5313) (width 2.5) (layer "B.Cu") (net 5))
 (segment locked (start 81.25 20.75) (end 81.25 12.0019) (width 2.5) (layer "B.Cu") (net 5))
 (segment locked (start 80.05 7.25) (end 80.05 10.8019) (width 2.5) (layer "B.Cu") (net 5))
 (segment (start 116.9251 85.8704) (end 118.9996 85.8704) (width 1.5998) (layer "B.Cu") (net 5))
 (segment (start 113.71 70.5) (end 114.586 71.376) (width 2.5) (layer "B.Cu") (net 5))
 (segment (start 109.17 28.5) (end 110.5 27.17) (width 2.5) (layer "B.Cu") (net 5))
 (segment locked (start 81.25 12.0019) (end 80.05 10.8019) (width 2.5) (layer "B.Cu") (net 5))
 (segment (start 109.17 28.5) (end 113.71 33.04) (width 2.5) (layer "B.Cu") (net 5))
 (segment (start 114.586 83.5313) (end 116.9251 85.8704) (width 2.5) (layer "B.Cu") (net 5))
 (segment (start 110.5 27.17) (end 110.5 19.25) (width 2.5) (layer "B.Cu") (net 5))
 (segment (start 113.71 33.04) (end 113.71 70.5) (width 2.5) (layer "B.Cu") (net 5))
 (segment (start 118.9996 85.8704) (end 119.31 85.56) (width 1.5998) (layer "B.Cu") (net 5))
 (segment (start 139.33 85.25) (end 132.02 77.94) (width 0.5) (layer "F.Cu") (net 8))
 (segment (start 132.02 77.94) (end 119.31 77.94) (width 0.5) (layer "F.Cu") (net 8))
 (segment (start 139.33 85.25) (end 144.2281 90.1481) (width 0.5) (layer "B.Cu") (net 8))
 (segment (start 124.499 81.0209) (end 124.499 99.501) (width 0.5) (layer "B.Cu") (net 8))
 (segment (start 144.2281 90.1481) (end 145.62 90.1481) (width 0.5) (layer "B.Cu") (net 8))
 (segment (start 121.4181 77.94) (end 124.499 81.0209) (width 0.5) (layer "B.Cu") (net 8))
 (segment (start 124.499 99.501) (end 118.75 105.25) (width 0.5) (layer "B.Cu") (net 8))
 (segment (start 119.31 77.94) (end 121.4181 77.94) (width 0.5) (layer "B.Cu") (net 8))
 (segment (start 145.62 92.5) (end 145.62 90.1481) (width 0.5) (layer "B.Cu") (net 8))
 (segment (start 127.1181 85.25) (end 122.3481 80.48) (width 0.5) (layer "F.Cu") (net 7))
 (segment (start 117.4581 80.48) (end 117.4581 71.8319) (width 0.5) (layer "F.Cu") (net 7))
 (segment (start 119.31 80.48) (end 117.4581 80.48) (width 0.5) (layer "F.Cu") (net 7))
 (segment (start 117.4581 71.8319) (end 118.79 70.5) (width 0.5) (layer "F.Cu") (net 7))
 (segment (start 129.17 85.25) (end 127.1181 85.25) (width 0.5) (layer "F.Cu") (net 7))
 (segment (start 122.3481 80.48) (end 119.31 80.48) (width 0.5) (layer "F.Cu") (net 7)))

